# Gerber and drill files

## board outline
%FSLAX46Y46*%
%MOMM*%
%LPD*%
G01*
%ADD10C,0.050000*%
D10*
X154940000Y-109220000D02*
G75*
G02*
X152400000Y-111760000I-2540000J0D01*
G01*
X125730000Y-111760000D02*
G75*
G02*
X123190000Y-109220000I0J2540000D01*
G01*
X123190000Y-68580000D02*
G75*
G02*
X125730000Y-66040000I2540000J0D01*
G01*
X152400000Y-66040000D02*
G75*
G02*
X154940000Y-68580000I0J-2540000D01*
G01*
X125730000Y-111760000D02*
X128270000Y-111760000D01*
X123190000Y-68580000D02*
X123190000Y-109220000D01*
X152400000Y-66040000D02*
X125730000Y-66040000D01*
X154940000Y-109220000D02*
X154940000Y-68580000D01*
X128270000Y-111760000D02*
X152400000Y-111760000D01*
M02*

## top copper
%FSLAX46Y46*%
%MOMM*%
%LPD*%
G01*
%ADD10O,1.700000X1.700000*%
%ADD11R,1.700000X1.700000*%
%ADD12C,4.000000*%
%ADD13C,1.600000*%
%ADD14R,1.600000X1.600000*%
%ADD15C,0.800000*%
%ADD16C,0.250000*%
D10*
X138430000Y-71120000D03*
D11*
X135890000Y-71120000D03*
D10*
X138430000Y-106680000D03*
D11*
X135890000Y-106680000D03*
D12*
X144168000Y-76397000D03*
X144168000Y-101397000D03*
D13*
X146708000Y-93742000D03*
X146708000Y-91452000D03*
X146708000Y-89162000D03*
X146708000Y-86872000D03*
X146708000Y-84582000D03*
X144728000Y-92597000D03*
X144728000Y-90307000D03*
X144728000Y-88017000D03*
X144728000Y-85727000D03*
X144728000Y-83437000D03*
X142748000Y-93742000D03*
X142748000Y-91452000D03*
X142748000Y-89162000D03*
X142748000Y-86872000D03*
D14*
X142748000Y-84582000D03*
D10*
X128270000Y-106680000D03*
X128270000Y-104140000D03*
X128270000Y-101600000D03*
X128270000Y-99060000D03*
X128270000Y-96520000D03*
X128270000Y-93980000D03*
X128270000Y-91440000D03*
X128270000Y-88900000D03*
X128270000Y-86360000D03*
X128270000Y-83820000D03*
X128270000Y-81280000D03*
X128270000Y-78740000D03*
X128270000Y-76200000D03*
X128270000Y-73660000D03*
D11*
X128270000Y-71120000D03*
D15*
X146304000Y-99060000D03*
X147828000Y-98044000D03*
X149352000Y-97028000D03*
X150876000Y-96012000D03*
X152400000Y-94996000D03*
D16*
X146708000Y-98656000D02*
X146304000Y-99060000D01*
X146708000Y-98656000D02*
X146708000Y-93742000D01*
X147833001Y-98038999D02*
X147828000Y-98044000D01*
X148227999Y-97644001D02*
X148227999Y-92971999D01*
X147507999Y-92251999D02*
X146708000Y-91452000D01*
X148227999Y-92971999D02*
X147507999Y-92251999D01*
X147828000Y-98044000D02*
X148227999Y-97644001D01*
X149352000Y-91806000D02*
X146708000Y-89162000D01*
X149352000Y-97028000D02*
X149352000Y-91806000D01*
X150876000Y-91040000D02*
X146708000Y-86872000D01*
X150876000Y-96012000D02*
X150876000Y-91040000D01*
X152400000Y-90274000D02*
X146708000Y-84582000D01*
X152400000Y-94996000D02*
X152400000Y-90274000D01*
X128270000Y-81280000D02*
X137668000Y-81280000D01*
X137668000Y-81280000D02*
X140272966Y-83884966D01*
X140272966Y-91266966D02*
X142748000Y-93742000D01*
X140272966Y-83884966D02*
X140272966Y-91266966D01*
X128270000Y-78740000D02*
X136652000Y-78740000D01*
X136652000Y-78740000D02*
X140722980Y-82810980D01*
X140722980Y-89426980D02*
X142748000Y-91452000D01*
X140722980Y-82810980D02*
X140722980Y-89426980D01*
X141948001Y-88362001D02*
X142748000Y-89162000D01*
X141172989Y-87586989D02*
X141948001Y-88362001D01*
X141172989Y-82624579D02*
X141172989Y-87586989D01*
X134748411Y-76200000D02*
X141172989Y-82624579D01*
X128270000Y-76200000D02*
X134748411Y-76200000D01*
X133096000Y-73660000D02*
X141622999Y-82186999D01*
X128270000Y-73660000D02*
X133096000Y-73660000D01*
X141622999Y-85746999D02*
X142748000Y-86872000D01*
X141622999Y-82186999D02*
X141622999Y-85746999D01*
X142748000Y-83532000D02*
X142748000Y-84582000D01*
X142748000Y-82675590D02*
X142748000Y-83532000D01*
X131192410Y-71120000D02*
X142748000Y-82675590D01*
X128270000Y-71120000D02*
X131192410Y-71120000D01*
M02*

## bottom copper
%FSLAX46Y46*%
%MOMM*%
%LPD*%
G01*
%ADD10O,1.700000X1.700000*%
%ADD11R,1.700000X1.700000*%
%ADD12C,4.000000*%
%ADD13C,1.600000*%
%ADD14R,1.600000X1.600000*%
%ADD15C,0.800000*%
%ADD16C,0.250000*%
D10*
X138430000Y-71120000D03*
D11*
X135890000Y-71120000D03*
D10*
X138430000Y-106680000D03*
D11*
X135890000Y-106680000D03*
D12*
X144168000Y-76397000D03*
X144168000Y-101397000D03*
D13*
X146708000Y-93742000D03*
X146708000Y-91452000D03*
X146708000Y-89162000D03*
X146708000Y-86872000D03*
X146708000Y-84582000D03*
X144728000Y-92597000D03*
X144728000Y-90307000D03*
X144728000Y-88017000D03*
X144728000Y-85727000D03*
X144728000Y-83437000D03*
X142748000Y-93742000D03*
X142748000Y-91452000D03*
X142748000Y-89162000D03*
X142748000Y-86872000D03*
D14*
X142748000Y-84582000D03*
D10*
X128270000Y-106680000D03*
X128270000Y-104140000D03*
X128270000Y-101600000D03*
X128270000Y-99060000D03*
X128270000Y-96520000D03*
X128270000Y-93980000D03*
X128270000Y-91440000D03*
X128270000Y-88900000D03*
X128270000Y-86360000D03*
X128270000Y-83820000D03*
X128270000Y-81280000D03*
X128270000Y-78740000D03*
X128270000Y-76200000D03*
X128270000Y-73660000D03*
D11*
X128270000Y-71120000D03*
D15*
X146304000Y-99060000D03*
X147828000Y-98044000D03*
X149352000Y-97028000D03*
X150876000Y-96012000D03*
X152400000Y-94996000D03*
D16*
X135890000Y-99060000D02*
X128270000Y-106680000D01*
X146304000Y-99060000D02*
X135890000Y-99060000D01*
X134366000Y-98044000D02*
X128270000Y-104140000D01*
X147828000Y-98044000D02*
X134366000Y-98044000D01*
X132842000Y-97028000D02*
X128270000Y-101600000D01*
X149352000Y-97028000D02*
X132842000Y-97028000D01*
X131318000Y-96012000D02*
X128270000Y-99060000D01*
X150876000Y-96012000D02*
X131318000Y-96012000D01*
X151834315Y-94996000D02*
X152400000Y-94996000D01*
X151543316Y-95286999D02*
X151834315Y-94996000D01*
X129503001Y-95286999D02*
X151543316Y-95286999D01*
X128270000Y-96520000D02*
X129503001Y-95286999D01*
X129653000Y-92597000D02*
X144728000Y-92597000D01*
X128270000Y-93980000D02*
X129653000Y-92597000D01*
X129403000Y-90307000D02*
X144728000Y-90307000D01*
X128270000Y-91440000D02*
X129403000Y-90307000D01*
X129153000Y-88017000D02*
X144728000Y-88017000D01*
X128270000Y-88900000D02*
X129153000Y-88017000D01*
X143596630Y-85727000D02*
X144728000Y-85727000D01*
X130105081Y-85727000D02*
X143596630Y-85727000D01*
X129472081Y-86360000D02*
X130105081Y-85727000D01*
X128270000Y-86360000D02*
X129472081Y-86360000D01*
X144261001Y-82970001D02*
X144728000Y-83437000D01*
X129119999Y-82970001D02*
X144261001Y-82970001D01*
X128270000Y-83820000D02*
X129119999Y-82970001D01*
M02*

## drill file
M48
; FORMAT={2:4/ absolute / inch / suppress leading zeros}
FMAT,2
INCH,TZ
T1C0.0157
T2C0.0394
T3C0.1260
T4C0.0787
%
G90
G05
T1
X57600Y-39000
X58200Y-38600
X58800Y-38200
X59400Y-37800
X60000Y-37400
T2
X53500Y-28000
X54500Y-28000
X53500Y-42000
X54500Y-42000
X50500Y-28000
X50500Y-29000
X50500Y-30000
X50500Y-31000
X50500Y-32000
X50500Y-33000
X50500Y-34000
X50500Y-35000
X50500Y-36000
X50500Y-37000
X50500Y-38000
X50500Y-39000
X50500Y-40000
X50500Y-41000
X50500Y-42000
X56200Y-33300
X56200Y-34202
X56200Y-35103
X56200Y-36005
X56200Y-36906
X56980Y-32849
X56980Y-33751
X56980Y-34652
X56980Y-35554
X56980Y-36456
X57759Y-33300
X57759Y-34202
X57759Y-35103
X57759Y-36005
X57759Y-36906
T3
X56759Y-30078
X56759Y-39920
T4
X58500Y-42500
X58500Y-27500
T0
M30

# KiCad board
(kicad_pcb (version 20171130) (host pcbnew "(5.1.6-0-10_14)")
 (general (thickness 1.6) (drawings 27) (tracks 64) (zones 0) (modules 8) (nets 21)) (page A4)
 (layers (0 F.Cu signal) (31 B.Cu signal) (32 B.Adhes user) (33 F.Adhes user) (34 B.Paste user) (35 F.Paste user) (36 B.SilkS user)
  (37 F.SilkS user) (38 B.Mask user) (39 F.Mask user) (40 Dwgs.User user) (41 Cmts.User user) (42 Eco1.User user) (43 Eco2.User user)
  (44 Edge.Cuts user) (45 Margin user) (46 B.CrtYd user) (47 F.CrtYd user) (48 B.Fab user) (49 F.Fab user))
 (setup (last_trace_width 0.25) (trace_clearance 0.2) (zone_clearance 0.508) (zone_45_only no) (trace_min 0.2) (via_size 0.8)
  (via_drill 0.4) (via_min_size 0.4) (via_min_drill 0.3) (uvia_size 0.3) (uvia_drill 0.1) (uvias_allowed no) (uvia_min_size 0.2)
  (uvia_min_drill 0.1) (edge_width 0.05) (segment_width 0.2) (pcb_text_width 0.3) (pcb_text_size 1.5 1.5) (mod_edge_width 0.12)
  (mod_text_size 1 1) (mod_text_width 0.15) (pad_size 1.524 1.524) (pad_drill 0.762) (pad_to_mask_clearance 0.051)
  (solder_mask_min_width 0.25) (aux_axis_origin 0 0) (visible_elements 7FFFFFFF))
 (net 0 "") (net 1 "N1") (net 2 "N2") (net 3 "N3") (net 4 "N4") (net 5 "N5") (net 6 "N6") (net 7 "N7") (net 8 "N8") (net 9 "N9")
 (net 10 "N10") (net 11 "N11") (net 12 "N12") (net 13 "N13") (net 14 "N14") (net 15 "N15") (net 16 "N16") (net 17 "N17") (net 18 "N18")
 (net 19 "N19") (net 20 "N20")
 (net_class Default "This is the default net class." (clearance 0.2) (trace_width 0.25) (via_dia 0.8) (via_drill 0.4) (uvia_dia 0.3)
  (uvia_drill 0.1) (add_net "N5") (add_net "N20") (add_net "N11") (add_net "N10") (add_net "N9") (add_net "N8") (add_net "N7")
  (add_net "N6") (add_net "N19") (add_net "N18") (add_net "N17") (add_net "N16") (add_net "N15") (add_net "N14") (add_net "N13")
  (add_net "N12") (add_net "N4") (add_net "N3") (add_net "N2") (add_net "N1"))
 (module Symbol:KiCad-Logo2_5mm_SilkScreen (layer B.Cu) (at 133.35 88.9 90)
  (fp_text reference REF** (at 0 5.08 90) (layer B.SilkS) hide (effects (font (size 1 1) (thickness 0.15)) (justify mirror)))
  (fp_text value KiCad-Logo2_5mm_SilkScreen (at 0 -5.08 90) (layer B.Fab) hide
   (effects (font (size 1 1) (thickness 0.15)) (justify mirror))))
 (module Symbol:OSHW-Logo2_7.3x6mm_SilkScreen (layer B.Cu) (at 151.13 88.9 90)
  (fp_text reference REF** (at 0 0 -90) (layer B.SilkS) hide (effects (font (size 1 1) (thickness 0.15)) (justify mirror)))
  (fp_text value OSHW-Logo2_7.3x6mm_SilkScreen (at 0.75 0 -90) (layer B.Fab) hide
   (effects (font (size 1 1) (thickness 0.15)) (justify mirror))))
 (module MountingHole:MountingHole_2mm (layer F.Cu) (at 148.59 107.95 90)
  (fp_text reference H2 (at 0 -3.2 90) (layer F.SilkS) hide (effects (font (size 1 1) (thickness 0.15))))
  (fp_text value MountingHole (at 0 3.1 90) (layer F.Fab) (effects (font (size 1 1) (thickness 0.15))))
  (pad "" np_thru_hole circle (at 0 0 90) (size 2 2) (drill 2) (layers *.Cu *.Mask)))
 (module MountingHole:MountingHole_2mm (layer F.Cu) (at 148.59 69.85 90)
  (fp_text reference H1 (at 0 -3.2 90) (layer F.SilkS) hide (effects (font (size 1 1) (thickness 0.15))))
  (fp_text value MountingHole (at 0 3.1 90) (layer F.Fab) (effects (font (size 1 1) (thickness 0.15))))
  (pad "" np_thru_hole circle (at 0 0 90) (size 2 2) (drill 2) (layers *.Cu *.Mask)))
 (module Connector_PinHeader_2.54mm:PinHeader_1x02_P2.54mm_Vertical (layer B.Cu) (at 135.89 71.12 270)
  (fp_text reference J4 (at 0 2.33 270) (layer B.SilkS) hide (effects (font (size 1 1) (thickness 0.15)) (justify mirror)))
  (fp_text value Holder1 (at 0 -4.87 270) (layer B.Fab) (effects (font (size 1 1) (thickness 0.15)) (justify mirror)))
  (pad 2 thru_hole oval (at 0 -2.54 270) (size 1.7 1.7) (drill 1) (layers *.Cu *.Mask) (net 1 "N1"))
  (pad 1 thru_hole rect (at 0 0 270) (size 1.7 1.7) (drill 1) (layers *.Cu *.Mask) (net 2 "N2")))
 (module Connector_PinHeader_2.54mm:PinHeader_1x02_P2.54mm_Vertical (layer B.Cu) (at 135.89 106.68 270)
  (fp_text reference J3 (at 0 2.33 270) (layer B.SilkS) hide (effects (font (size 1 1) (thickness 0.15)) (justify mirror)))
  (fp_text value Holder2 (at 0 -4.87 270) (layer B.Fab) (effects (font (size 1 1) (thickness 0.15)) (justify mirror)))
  (pad 2 thru_hole oval (at 0 -2.54 270) (size 1.7 1.7) (drill 1) (layers *.Cu *.Mask) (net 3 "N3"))
  (pad 1 thru_hole rect (at 0 0 270) (size 1.7 1.7) (drill 1) (layers *.Cu *.Mask) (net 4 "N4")))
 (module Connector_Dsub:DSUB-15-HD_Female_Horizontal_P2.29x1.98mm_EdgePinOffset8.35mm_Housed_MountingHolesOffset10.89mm (layer F.Cu)
  (at 142.748 84.582 90)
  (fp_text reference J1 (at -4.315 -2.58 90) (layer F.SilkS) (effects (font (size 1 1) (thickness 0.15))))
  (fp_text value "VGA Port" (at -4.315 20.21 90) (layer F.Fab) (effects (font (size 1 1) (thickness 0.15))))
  (pad 0 thru_hole circle (at 8.185 1.42 90) (size 4 4) (drill 3.2) (layers *.Cu *.Mask) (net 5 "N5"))
  (pad 0 thru_hole circle (at -16.815 1.42 90) (size 4 4) (drill 3.2) (layers *.Cu *.Mask) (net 5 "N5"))
  (pad 15 thru_hole circle (at -9.16 3.96 90) (size 1.6 1.6) (drill 1) (layers *.Cu *.Mask) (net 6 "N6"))
  (pad 14 thru_hole circle (at -6.87 3.96 90) (size 1.6 1.6) (drill 1) (layers *.Cu *.Mask) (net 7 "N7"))
  (pad 13 thru_hole circle (at -4.58 3.96 90) (size 1.6 1.6) (drill 1) (layers *.Cu *.Mask) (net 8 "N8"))
  (pad 12 thru_hole circle (at -2.29 3.96 90) (size 1.6 1.6) (drill 1) (layers *.Cu *.Mask) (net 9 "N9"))
  (pad 11 thru_hole circle (at 0 3.96 90) (size 1.6 1.6) (drill 1) (layers *.Cu *.Mask) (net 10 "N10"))
  (pad 10 thru_hole circle (at -8.015 1.98 90) (size 1.6 1.6) (drill 1) (layers *.Cu *.Mask) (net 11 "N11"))
  (pad 9 thru_hole circle (at -5.725 1.98 90) (size 1.6 1.6) (drill 1) (layers *.Cu *.Mask) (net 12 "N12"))
  (pad 8 thru_hole circle (at -3.435 1.98 90) (size 1.6 1.6) (drill 1) (layers *.Cu *.Mask) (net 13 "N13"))
  (pad 7 thru_hole circle (at -1.145 1.98 90) (size 1.6 1.6) (drill 1) (layers *.Cu *.Mask) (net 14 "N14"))
  (pad 6 thru_hole circle (at 1.145 1.98 90) (size 1.6 1.6) (drill 1) (layers *.Cu *.Mask) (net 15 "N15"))
  (pad 5 thru_hole circle (at -9.16 0 90) (size 1.6 1.6) (drill 1) (layers *.Cu *.Mask) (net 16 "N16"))
  (pad 4 thru_hole circle (at -6.87 0 90) (size 1.6 1.6) (drill 1) (layers *.Cu *.Mask) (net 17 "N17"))
  (pad 3 thru_hole circle (at -4.58 0 90) (size 1.6 1.6) (drill 1) (layers *.Cu *.Mask) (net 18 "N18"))
  (pad 2 thru_hole circle (at -2.29 0 90) (size 1.6 1.6) (drill 1) (layers *.Cu *.Mask) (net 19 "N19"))
  (pad 1 thru_hole rect (at 0 0 90) (size 1.6 1.6) (drill 1) (layers *.Cu *.Mask) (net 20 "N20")))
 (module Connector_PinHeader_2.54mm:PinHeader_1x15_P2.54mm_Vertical (layer B.Cu) (at 128.27 71.12 180)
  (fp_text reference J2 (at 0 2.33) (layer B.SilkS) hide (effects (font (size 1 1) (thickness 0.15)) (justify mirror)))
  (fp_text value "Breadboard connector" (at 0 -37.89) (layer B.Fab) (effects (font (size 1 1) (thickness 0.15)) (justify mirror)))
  (pad 15 thru_hole oval (at 0 -35.56 180) (size 1.7 1.7) (drill 1) (layers *.Cu *.Mask) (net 6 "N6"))
  (pad 14 thru_hole oval (at 0 -33.02 180) (size 1.7 1.7) (drill 1) (layers *.Cu *.Mask) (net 7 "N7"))
  (pad 13 thru_hole oval (at 0 -30.48 180) (size 1.7 1.7) (drill 1) (layers *.Cu *.Mask) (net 8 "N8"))
  (pad 12 thru_hole oval (at 0 -27.94 180) (size 1.7 1.7) (drill 1) (layers *.Cu *.Mask) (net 9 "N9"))
  (pad 11 thru_hole oval (at 0 -25.4 180) (size 1.7 1.7) (drill 1) (layers *.Cu *.Mask) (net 10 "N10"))
  (pad 10 thru_hole oval (at 0 -22.86 180) (size 1.7 1.7) (drill 1) (layers *.Cu *.Mask) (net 11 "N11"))
  (pad 9 thru_hole oval (at 0 -20.32 180) (size 1.7 1.7) (drill 1) (layers *.Cu *.Mask) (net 12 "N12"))
  (pad 8 thru_hole oval (at 0 -17.78 180) (size 1.7 1.7) (drill 1) (layers *.Cu *.Mask) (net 13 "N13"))
  (pad 7 thru_hole oval (at 0 -15.24 180) (size 1.7 1.7) (drill 1) (layers *.Cu *.Mask) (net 14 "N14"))
  (pad 6 thru_hole oval (at 0 -12.7 180) (size 1.7 1.7) (drill 1) (layers *.Cu *.Mask) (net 15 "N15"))
  (pad 5 thru_hole oval (at 0 -10.16 180) (size 1.7 1.7) (drill 1) (layers *.Cu *.Mask) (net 16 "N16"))
  (pad 4 thru_hole oval (at 0 -7.62 180) (size 1.7 1.7) (drill 1) (layers *.Cu *.Mask) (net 17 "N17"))
  (pad 3 thru_hole oval (at 0 -5.08 180) (size 1.7 1.7) (drill 1) (layers *.Cu *.Mask) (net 18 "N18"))
  (pad 2 thru_hole oval (at 0 -2.54 180) (size 1.7 1.7) (drill 1) (layers *.Cu *.Mask) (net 19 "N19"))
  (pad 1 thru_hole rect (at 0 0 180) (size 1.7 1.7) (drill 1) (layers *.Cu *.Mask) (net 20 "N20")))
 (gr_arc (start 152.4 109.22) (end 152.4 111.76) (angle -90) (layer Edge.Cuts) (width 0.05))
 (gr_arc (start 125.73 109.22) (end 123.19 109.22) (angle -90) (layer Edge.Cuts) (width 0.05))
 (gr_arc (start 125.73 68.58) (end 125.73 66.04) (angle -90) (layer Edge.Cuts) (width 0.05))
 (gr_arc (start 152.4 68.58) (end 154.94 68.58) (angle -90) (layer Edge.Cuts) (width 0.05))
 (gr_line (start 125.73 111.76) (end 128.27 111.76) (layer Edge.Cuts) (width 0.05))
 (gr_line (start 123.19 68.58) (end 123.19 109.22) (layer Edge.Cuts) (width 0.05))
 (gr_line (start 152.4 66.04) (end 125.73 66.04) (layer Edge.Cuts) (width 0.05))
 (gr_line (start 154.94 109.22) (end 154.94 68.58) (layer Edge.Cuts) (width 0.05))
 (gr_line (start 128.27 111.76) (end 152.4 111.76) (layer Edge.Cuts) (width 0.05))
 (via (at 146.304 99.06) (size 0.8) (drill 0.4) (layers F.Cu B.Cu) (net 6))
 (segment (start 146.708 98.656) (end 146.304 99.06) (width 0.25) (layer F.Cu) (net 6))
 (segment (start 135.89 99.06) (end 128.27 106.68) (width 0.25) (layer B.Cu) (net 6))
 (segment (start 146.304 99.06) (end 135.89 99.06) (width 0.25) (layer B.Cu) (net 6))
 (segment (start 146.708 98.656) (end 146.708 93.742) (width 0.25) (layer F.Cu) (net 6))
 (via (at 147.828 98.044) (size 0.8) (drill 0.4) (layers F.Cu B.Cu) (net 7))
 (segment (start 147.833001 98.038999) (end 147.828 98.044) (width 0.25) (layer F.Cu) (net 7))
 (segment (start 134.366 98.044) (end 128.27 104.14) (width 0.25) (layer B.Cu) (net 7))
 (segment (start 147.828 98.044) (end 134.366 98.044) (width 0.25) (layer B.Cu) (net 7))
 (segment (start 148.227999 97.644001) (end 148.227999 92.971999) (width 0.25) (layer F.Cu) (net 7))
 (segment (start 147.507999 92.251999) (end 146.708 91.452) (width 0.25) (layer F.Cu) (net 7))
 (segment (start 148.227999 92.971999) (end 147.507999 92.251999) (width 0.25) (layer F.Cu) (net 7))
 (segment (start 147.828 98.044) (end 148.227999 97.644001) (width 0.25) (layer F.Cu) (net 7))
 (via (at 149.352 97.028) (size 0.8) (drill 0.4) (layers F.Cu B.Cu) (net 8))
 (segment (start 132.842 97.028) (end 128.27 101.6) (width 0.25) (layer B.Cu) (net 8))
 (segment (start 149.352 97.028) (end 132.842 97.028) (width 0.25) (layer B.Cu) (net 8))
 (segment (start 149.352 91.806) (end 146.708 89.162) (width 0.25) (layer F.Cu) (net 8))
 (segment (start 149.352 97.028) (end 149.352 91.806) (width 0.25) (layer F.Cu) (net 8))
 (via (at 150.876 96.012) (size 0.8) (drill 0.4) (layers F.Cu B.Cu) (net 9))
 (segment (start 131.318 96.012) (end 128.27 99.06) (width 0.25) (layer B.Cu) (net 9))
 (segment (start 150.876 96.012) (end 131.318 96.012) (width 0.25) (layer B.Cu) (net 9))
 (segment (start 150.876 91.04) (end 146.708 86.872) (width 0.25) (layer F.Cu) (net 9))
 (segment (start 150.876 96.012) (end 150.876 91.04) (width 0.25) (layer F.Cu) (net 9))
 (via (at 152.4 94.996) (size 0.8) (drill 0.4) (layers F.Cu B.Cu) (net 10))
 (segment (start 151.834315 94.996) (end 152.4 94.996) (width 0.25) (layer B.Cu) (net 10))
 (segment (start 151.543316 95.286999) (end 151.834315 94.996) (width 0.25) (layer B.Cu) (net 10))
 (segment (start 129.503001 95.286999) (end 151.543316 95.286999) (width 0.25) (layer B.Cu) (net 10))
 (segment (start 128.27 96.52) (end 129.503001 95.286999) (width 0.25) (layer B.Cu) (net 10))
 (segment (start 152.4 90.274) (end 146.708 84.582) (width 0.25) (layer F.Cu) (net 10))
 (segment (start 152.4 94.996) (end 152.4 90.274) (width 0.25) (layer F.Cu) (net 10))
 (segment (start 129.653 92.597) (end 144.728 92.597) (width 0.25) (layer B.Cu) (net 11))
 (segment (start 128.27 93.98) (end 129.653 92.597) (width 0.25) (layer B.Cu) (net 11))
 (segment (start 129.403 90.307) (end 144.728 90.307) (width 0.25) (layer B.Cu) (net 12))
 (segment (start 128.27 91.44) (end 129.403 90.307) (width 0.25) (layer B.Cu) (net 12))
 (segment (start 129.153 88.017) (end 144.728 88.017) (width 0.25) (layer B.Cu) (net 13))
 (segment (start 128.27 88.9) (end 129.153 88.017) (width 0.25) (layer B.Cu) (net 13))
 (segment (start 143.59663 85.727) (end 144.728 85.727) (width 0.25) (layer B.Cu) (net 14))
 (segment (start 130.105081 85.727) (end 143.59663 85.727) (width 0.25) (layer B.Cu) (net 14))
 (segment (start 129.472081 86.36) (end 130.105081 85.727) (width 0.25) (layer B.Cu) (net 14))
 (segment (start 128.27 86.36) (end 129.472081 86.36) (width 0.25) (layer B.Cu) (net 14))
 (segment (start 144.261001 82.970001) (end 144.728 83.437) (width 0.25) (layer B.Cu) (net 15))
 (segment (start 129.119999 82.970001) (end 144.261001 82.970001) (width 0.25) (layer B.Cu) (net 15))
 (segment (start 128.27 83.82) (end 129.119999 82.970001) (width 0.25) (layer B.Cu) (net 15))
 (segment (start 128.27 81.28) (end 137.668 81.28) (width 0.25) (layer F.Cu) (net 16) (status 10))
 (segment (start 137.668 81.28) (end 140.272966 83.884966) (width 0.25) (layer F.Cu) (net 16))
 (segment (start 140.272966 91.266966) (end 142.748 93.742) (width 0.25) (layer F.Cu) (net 16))
 (segment (start 140.272966 83.884966) (end 140.272966 91.266966) (width 0.25) (layer F.Cu) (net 16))
 (segment (start 128.27 78.74) (end 136.652 78.74) (width 0.25) (layer F.Cu) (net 17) (status 10))
 (segment (start 136.652 78.74) (end 140.72298 82.81098) (width 0.25) (layer F.Cu) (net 17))
 (segment (start 140.72298 89.42698) (end 142.748 91.452) (width 0.25) (layer F.Cu) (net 17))
 (segment (start 140.72298 82.81098) (end 140.72298 89.42698) (width 0.25) (layer F.Cu) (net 17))
 (segment (start 141.948001 88.362001) (end 142.748 89.162) (width 0.25) (layer F.Cu) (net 18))
 (segment (start 141.172989 87.586989) (end 141.948001 88.362001) (width 0.25) (layer F.Cu) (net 18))
 (segment (start 141.172989 82.624579) (end 141.172989 87.586989) (width 0.25) (layer F.Cu) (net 18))
 (segment (start 134.748411 76.2) (end 141.172989 82.624579) (width 0.25) (layer F.Cu) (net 18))
 (segment (start 128.27 76.2) (end 134.748411 76.2) (width 0.25) (layer F.Cu) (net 18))
 (segment (start 133.096 73.66) (end 141.622999 82.186999) (width 0.25) (layer F.Cu) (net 19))
 (segment (start 128.27 73.66) (end 133.096 73.66) (width 0.25) (layer F.Cu) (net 19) (status 10))
 (segment (start 141.622999 85.746999) (end 142.748 86.872) (width 0.25) (layer F.Cu) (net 19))
 (segment (start 141.622999 82.186999) (end 141.622999 85.746999) (width 0.25) (layer F.Cu) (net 19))
 (segment (start 142.748 83.532) (end 142.748 84.582) (width 0.25) (layer F.Cu) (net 20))
 (segment (start 142.748 82.67559) (end 142.748 83.532) (width 0.25) (layer F.Cu) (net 20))
 (segment (start 131.19241 71.12) (end 142.748 82.67559) (width 0.25) (layer F.Cu) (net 20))
 (segment (start 128.27 71.12) (end 131.19241 71.12) (width 0.25) (layer F.Cu) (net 20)))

